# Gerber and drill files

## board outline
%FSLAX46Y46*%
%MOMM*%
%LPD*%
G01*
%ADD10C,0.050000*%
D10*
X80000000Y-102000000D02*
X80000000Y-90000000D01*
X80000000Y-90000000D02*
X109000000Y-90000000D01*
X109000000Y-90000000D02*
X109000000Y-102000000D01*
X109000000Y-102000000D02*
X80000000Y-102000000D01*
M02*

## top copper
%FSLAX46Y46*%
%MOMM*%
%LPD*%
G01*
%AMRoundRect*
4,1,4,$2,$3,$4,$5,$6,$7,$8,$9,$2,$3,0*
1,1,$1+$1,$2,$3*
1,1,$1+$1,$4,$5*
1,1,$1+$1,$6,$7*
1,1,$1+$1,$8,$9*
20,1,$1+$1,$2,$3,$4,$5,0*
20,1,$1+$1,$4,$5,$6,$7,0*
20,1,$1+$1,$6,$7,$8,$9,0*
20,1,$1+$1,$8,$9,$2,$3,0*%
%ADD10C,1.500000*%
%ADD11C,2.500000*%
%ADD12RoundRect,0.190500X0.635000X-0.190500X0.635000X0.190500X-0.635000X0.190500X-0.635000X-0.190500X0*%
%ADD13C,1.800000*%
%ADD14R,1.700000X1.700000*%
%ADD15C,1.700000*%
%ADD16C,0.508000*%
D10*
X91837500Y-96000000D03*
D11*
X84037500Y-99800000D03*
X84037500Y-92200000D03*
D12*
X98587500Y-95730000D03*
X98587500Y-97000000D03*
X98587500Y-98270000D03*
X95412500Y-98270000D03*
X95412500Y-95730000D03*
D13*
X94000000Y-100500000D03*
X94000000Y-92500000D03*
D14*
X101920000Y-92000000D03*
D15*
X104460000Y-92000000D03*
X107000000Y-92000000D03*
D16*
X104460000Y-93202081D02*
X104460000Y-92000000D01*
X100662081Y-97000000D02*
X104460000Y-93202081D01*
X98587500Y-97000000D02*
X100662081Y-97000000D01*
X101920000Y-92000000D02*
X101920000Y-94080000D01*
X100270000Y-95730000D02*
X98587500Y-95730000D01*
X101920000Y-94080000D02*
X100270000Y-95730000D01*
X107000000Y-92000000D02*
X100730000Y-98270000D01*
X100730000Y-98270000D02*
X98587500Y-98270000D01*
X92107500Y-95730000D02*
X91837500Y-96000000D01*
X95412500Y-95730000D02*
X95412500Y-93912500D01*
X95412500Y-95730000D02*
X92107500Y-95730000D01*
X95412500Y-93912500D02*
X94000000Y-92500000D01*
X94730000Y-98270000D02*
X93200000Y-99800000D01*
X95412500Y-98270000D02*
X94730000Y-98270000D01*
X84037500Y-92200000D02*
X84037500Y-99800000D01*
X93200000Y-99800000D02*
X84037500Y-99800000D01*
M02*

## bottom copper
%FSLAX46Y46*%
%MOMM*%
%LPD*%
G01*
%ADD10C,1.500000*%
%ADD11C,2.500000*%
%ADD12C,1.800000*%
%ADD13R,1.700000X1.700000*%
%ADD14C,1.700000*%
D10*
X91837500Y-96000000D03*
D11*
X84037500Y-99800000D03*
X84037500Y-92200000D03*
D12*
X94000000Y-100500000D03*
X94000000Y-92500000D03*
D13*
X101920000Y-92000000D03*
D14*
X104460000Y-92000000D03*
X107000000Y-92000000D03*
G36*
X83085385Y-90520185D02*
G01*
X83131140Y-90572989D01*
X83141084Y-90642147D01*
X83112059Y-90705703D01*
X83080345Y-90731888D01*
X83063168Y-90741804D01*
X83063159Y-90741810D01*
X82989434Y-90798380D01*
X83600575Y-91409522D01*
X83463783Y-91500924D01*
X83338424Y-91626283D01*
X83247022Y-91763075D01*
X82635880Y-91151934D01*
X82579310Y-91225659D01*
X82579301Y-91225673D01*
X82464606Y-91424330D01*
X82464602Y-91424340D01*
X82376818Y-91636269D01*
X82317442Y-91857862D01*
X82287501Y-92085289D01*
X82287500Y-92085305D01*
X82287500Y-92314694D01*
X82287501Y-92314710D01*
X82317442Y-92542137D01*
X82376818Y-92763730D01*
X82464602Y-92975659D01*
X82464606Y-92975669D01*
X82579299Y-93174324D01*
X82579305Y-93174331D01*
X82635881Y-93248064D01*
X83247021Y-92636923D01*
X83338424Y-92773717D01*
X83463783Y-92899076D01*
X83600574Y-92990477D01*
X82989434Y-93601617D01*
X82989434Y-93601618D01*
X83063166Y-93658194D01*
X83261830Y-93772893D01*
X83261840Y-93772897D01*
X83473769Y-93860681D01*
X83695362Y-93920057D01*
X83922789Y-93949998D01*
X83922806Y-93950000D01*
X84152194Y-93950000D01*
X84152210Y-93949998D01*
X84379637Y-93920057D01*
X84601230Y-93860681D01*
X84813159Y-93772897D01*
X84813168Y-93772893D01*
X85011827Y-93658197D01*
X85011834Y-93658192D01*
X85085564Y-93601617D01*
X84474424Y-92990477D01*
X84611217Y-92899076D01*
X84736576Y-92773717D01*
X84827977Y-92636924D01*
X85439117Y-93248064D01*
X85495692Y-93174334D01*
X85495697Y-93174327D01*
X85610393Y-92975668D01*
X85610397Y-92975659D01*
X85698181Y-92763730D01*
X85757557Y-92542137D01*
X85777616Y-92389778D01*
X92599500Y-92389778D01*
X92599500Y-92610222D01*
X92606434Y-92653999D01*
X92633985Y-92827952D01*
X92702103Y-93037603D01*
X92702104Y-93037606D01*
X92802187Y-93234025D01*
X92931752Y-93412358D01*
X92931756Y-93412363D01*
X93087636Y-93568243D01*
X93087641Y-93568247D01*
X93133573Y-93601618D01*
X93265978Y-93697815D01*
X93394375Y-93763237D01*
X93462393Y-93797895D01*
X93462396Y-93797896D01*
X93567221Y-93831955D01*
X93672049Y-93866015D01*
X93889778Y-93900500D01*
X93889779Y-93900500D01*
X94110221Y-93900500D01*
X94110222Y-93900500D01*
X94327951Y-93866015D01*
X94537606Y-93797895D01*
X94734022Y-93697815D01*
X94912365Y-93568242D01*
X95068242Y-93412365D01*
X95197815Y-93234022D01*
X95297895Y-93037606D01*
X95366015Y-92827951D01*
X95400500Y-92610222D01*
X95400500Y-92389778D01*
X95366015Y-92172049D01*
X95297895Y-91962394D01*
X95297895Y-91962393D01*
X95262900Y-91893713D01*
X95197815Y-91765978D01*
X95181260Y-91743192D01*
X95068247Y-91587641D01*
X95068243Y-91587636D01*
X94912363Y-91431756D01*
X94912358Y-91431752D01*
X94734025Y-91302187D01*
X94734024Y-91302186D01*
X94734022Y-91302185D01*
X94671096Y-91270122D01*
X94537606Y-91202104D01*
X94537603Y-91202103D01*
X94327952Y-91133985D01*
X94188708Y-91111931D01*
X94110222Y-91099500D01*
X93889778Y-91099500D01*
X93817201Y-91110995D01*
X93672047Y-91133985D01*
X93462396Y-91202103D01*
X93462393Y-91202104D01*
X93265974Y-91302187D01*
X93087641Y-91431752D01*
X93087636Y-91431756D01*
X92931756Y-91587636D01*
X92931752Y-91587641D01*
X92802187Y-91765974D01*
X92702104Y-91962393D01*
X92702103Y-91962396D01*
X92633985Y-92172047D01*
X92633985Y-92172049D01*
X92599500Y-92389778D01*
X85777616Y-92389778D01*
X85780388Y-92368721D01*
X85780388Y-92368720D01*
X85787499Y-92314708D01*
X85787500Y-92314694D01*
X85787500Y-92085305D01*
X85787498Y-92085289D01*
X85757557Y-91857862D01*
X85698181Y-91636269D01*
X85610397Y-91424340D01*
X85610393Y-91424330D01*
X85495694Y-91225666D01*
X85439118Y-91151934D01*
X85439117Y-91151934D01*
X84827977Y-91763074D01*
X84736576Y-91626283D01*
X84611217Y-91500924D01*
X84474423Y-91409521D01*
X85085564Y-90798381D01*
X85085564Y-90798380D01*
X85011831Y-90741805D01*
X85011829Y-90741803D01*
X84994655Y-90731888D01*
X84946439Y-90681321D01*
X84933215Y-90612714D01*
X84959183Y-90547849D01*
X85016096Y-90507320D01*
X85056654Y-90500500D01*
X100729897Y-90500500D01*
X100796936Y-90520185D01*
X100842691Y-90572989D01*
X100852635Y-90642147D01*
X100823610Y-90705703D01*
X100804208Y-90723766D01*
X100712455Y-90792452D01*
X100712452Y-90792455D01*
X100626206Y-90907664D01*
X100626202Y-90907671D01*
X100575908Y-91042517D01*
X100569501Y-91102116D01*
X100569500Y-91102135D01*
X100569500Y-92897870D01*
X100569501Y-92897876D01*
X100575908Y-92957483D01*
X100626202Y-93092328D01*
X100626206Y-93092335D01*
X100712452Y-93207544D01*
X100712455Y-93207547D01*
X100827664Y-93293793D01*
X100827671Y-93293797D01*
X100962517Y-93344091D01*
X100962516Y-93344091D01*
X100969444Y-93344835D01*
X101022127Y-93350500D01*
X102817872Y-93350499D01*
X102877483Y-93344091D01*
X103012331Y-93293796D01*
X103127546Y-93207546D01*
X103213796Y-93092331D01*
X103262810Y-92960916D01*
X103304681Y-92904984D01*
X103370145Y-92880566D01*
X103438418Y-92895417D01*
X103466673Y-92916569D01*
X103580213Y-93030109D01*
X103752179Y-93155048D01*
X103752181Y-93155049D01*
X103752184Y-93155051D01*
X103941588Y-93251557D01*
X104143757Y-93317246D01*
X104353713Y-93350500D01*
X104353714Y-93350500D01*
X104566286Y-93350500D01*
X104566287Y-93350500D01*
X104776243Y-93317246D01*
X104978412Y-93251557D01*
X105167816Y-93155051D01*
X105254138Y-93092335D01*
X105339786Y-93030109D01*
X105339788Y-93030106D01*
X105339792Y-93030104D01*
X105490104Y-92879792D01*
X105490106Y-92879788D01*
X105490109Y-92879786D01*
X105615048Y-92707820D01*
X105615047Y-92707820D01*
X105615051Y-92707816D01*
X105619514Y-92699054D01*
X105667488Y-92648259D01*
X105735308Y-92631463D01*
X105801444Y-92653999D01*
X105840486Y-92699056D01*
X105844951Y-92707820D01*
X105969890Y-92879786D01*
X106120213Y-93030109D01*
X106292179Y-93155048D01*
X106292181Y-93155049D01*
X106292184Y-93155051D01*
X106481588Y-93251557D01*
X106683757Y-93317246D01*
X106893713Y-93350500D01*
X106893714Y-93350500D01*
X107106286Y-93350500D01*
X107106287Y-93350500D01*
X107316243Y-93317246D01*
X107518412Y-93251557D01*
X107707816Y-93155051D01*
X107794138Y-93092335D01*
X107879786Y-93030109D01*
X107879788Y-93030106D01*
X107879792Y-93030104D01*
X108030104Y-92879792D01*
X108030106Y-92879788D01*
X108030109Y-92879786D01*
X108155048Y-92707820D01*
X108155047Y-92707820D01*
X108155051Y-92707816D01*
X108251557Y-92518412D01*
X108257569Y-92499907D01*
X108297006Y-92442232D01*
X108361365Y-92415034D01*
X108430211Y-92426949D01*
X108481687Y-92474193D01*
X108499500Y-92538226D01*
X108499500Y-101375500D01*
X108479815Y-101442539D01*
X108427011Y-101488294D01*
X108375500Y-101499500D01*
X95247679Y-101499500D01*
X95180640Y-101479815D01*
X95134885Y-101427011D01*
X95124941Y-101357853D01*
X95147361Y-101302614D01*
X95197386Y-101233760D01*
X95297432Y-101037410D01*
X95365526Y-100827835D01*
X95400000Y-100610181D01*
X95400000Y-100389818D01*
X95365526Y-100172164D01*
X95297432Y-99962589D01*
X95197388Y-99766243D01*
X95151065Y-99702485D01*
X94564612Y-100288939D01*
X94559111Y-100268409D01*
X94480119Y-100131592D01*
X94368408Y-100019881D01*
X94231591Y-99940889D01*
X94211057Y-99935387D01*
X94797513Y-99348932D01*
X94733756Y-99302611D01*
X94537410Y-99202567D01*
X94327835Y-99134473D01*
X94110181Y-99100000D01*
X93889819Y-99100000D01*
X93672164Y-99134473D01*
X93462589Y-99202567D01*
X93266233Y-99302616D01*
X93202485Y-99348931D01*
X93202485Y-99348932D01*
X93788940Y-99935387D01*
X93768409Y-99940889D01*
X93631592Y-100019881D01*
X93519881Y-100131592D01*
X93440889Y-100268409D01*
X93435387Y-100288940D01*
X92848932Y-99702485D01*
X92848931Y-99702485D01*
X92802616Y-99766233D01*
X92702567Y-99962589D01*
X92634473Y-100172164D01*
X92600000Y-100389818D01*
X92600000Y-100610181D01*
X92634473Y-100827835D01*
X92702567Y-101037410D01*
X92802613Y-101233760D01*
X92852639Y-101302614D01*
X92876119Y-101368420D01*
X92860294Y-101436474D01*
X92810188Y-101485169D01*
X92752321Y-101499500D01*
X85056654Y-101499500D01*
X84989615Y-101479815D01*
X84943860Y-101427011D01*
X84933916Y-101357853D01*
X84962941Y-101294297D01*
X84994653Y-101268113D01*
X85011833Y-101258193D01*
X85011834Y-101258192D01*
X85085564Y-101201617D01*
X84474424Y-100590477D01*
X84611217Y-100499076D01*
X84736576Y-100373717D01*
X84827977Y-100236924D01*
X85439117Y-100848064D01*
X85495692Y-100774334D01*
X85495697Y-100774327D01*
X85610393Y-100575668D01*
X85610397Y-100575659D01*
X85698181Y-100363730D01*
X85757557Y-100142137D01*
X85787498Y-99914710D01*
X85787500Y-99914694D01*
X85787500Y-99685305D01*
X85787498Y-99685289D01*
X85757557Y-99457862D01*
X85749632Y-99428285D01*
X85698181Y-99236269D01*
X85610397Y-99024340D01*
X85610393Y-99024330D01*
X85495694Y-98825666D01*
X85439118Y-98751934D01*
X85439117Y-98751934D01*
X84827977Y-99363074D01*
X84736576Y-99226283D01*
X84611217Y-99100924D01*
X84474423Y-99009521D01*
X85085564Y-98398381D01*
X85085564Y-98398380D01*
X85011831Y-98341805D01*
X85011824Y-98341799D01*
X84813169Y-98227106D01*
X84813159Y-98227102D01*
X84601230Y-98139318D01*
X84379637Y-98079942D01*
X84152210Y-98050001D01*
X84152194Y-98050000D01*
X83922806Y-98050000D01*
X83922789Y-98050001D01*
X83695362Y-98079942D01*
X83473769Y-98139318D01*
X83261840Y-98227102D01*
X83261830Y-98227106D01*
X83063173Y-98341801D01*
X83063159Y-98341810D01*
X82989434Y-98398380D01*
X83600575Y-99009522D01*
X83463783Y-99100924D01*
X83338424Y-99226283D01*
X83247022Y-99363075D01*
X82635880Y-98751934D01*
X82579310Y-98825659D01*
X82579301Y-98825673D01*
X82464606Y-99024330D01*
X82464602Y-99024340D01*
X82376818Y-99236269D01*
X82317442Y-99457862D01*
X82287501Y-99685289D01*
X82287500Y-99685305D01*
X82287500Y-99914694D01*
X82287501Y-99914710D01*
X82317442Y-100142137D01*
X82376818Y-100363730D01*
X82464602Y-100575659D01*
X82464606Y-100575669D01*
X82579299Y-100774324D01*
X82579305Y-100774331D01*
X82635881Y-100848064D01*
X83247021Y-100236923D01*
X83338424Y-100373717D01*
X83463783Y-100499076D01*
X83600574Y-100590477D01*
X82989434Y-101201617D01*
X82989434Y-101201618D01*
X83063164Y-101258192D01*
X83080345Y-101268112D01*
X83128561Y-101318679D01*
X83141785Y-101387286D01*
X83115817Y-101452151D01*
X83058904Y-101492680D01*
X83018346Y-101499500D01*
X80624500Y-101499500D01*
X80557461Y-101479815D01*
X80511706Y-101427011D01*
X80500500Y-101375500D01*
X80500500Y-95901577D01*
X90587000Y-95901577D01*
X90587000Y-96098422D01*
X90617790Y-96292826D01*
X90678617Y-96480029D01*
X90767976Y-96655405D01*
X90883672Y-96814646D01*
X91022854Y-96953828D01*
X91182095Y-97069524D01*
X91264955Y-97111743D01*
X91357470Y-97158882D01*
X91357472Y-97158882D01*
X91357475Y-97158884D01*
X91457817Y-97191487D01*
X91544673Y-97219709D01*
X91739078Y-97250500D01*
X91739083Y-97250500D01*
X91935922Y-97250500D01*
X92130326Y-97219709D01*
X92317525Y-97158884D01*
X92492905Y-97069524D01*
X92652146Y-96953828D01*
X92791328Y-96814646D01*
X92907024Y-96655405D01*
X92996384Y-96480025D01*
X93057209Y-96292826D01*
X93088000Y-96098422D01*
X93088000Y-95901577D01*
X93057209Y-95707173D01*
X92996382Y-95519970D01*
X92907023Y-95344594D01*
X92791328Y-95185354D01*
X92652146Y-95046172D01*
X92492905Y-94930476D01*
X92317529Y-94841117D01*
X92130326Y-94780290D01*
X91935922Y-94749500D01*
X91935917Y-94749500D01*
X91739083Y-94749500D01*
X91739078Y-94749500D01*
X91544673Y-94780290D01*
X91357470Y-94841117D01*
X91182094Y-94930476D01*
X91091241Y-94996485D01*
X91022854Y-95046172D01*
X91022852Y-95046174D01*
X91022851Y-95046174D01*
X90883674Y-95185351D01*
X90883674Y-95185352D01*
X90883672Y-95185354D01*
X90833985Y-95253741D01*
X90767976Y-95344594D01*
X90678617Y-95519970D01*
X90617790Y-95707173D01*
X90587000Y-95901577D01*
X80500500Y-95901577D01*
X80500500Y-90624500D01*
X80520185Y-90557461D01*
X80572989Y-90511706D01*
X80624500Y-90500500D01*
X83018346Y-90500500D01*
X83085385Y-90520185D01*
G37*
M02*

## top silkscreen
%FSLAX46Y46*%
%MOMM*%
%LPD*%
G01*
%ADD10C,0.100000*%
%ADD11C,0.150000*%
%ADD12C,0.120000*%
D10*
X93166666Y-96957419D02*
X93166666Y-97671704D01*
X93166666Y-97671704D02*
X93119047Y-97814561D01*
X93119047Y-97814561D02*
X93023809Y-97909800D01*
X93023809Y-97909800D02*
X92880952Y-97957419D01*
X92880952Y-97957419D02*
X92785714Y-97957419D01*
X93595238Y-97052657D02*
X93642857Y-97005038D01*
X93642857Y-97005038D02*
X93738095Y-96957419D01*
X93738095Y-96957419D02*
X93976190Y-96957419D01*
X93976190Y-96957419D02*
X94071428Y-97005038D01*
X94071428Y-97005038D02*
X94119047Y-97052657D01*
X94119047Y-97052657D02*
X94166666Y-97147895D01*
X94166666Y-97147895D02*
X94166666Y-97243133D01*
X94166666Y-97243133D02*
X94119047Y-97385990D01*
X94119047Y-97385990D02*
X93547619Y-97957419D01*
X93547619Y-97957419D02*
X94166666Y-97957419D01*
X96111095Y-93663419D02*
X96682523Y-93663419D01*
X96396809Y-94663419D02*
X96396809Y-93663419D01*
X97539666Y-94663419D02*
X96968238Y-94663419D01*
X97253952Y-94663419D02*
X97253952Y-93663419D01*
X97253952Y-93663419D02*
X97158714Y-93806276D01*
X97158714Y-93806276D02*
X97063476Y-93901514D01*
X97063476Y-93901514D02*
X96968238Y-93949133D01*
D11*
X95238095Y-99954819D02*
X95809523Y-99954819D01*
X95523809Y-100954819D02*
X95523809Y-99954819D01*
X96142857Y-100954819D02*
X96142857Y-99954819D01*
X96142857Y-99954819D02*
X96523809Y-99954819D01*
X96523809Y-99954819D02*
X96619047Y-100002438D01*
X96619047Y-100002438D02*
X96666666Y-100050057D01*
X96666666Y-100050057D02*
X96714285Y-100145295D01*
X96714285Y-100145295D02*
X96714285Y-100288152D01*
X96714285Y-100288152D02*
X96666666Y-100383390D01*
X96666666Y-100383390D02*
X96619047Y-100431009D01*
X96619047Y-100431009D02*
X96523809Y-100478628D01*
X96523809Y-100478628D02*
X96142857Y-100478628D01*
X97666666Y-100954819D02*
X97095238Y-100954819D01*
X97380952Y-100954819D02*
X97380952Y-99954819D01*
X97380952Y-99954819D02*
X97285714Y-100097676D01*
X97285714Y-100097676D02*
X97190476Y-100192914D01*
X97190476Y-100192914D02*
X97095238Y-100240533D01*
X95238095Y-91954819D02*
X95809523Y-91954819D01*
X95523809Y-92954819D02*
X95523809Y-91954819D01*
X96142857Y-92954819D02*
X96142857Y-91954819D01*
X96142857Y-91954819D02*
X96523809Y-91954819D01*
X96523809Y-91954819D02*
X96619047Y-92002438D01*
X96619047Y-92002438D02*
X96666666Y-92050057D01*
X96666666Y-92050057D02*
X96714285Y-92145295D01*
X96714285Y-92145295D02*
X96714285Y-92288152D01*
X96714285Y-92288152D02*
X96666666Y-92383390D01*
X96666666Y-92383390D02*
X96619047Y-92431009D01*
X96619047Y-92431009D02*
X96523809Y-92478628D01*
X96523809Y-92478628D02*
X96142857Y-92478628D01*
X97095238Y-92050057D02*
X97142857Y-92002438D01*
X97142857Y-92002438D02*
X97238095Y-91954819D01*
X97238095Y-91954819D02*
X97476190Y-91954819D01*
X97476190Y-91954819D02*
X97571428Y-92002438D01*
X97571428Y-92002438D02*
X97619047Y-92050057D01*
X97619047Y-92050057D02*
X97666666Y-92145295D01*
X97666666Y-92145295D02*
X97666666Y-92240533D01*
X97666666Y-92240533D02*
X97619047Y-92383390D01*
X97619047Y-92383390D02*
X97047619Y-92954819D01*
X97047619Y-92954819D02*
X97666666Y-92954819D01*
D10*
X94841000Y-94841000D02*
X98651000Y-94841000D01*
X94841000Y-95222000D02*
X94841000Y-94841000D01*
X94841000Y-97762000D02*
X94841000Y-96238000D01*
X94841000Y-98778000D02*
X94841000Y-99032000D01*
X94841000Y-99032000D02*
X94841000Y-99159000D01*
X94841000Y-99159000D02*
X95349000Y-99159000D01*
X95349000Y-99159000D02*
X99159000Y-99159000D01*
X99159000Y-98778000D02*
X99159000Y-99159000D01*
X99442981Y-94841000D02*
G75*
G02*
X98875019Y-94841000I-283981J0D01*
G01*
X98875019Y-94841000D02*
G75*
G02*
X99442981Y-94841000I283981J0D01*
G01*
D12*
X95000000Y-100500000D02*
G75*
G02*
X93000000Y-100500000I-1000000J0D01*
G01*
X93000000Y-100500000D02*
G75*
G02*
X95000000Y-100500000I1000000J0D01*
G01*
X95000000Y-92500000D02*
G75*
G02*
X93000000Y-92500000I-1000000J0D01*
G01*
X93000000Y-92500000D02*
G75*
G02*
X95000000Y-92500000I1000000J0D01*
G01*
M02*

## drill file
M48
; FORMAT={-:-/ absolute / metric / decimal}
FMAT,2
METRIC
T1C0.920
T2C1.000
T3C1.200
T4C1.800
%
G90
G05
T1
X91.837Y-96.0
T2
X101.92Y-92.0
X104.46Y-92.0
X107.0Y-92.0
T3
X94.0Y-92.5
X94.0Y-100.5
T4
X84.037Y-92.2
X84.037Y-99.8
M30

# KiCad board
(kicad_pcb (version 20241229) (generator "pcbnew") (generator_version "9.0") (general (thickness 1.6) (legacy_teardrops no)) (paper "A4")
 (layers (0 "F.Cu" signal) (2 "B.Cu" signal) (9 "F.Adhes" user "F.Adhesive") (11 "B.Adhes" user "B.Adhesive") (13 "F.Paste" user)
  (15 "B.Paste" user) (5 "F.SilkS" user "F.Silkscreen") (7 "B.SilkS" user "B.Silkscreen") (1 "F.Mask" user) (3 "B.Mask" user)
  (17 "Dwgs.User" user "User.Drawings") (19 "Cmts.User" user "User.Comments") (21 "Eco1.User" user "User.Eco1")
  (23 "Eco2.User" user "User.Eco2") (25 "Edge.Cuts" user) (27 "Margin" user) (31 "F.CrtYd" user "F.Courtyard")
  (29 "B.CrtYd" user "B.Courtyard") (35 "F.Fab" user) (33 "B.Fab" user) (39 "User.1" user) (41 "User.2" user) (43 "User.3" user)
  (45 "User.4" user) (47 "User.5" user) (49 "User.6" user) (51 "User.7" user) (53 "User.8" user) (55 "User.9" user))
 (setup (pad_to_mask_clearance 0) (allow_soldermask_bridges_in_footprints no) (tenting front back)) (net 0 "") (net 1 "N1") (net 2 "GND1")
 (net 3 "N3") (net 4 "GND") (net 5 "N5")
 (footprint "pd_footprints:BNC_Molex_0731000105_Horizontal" (layer "F.Cu") (at 84.0375 96 90)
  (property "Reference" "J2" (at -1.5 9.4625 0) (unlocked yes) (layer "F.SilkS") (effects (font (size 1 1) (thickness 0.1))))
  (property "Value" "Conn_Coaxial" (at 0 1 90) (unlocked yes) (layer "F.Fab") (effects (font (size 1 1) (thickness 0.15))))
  (pad "1" thru_hole circle (at 0 7.8 90) (size 1.5 1.5) (drill 0.92) (layers "*.Cu" "*.Mask") (remove_unused_layers no) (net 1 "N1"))
  (pad "2" thru_hole circle (at -3.8 0 90) (size 2.5 2.5) (drill 1.8) (layers "*.Cu" "*.Mask") (remove_unused_layers no) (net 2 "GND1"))
  (pad "2" thru_hole circle (at 3.8 0 90) (size 2.5 2.5) (drill 1.8) (layers "*.Cu" "*.Mask") (remove_unused_layers no) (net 2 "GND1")))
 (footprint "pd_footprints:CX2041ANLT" (layer "F.Cu") (at 97 97 90)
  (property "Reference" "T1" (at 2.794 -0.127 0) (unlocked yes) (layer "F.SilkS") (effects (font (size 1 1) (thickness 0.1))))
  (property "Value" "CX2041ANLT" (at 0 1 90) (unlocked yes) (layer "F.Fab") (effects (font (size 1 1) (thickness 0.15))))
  (fp_line (start 2.159 -2.159) (end 2.159 1.651) (stroke (width 0.1) (type default)) (layer "F.SilkS"))
  (fp_line (start 1.778 -2.159) (end 2.159 -2.159) (stroke (width 0.1) (type default)) (layer "F.SilkS"))
  (fp_line (start -0.762 -2.159) (end 0.762 -2.159) (stroke (width 0.1) (type default)) (layer "F.SilkS"))
  (fp_line (start -1.778 -2.159) (end -2.032 -2.159) (stroke (width 0.1) (type default)) (layer "F.SilkS"))
  (fp_line (start -2.032 -2.159) (end -2.159 -2.159) (stroke (width 0.1) (type default)) (layer "F.SilkS"))
  (fp_line (start -2.159 -2.159) (end -2.159 -1.651) (stroke (width 0.1) (type default)) (layer "F.SilkS"))
  (fp_line (start -2.159 -1.651) (end -2.159 2.159) (stroke (width 0.1) (type default)) (layer "F.SilkS"))
  (fp_line (start -1.778 2.159) (end -2.159 2.159) (stroke (width 0.1) (type default)) (layer "F.SilkS"))
  (fp_circle (center 2.159 2.159) (end 2.286 1.905) (stroke (width 0.1) (type default)) (fill no) (layer "F.SilkS"))
  (pad "1" smd roundrect (at 1.27 1.5875 90) (size 0.762 1.651) (layers "F.Cu" "F.Mask" "F.Paste") (roundrect_rratio 0.25) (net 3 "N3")
   (thermal_bridge_angle 45))
  (pad "2" smd roundrect (at 0 1.5875 90) (size 0.762 1.651) (layers "F.Cu" "F.Mask" "F.Paste") (roundrect_rratio 0.25) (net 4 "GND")
   (thermal_bridge_angle 45))
  (pad "3" smd roundrect (at -1.27 1.5875 90) (size 0.762 1.651) (layers "F.Cu" "F.Mask" "F.Paste") (roundrect_rratio 0.25) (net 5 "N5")
   (thermal_bridge_angle 45))
  (pad "4" smd roundrect (at -1.27 -1.5875 90) (size 0.762 1.651) (layers "F.Cu" "F.Mask" "F.Paste") (roundrect_rratio 0.25) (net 2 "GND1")
   (thermal_bridge_angle 45))
  (pad "6" smd roundrect (at 1.27 -1.5875 90) (size 0.762 1.651) (layers "F.Cu" "F.Mask" "F.Paste") (roundrect_rratio 0.25) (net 1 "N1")
   (thermal_bridge_angle 45)))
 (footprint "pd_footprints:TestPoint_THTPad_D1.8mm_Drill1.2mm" (layer "F.Cu") (at 94 100.5)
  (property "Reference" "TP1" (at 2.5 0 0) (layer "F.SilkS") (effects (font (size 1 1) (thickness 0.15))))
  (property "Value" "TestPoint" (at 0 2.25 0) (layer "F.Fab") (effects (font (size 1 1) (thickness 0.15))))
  (fp_circle (center 0 0) (end 1 0) (stroke (width 0.12) (type solid)) (fill no) (layer "F.SilkS"))
  (pad "1" thru_hole circle (at 0 0) (size 1.8 1.8) (drill 1.2) (layers "*.Cu" "*.Mask") (remove_unused_layers no) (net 2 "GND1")))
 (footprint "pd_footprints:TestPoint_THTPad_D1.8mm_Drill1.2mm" (layer "F.Cu") (at 94 92.5)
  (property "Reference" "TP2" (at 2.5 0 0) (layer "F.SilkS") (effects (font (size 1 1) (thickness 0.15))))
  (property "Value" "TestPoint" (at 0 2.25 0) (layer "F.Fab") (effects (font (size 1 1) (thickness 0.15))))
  (fp_circle (center 0 0) (end 1 0) (stroke (width 0.12) (type solid)) (fill no) (layer "F.SilkS"))
  (pad "1" thru_hole circle (at 0 0) (size 1.8 1.8) (drill 1.2) (layers "*.Cu" "*.Mask") (remove_unused_layers no) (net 1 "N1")))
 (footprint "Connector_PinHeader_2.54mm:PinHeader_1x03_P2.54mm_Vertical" (layer "B.Cu") (at 101.92 92 -90)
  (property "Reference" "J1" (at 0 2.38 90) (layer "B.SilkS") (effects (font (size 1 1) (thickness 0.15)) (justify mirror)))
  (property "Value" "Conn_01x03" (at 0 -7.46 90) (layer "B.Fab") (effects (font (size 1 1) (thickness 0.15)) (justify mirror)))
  (pad "1" thru_hole rect (at 0 0 270) (size 1.7 1.7) (drill 1) (layers "*.Cu" "*.Mask") (remove_unused_layers no) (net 3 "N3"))
  (pad "2" thru_hole circle (at 0 -2.54 270) (size 1.7 1.7) (drill 1) (layers "*.Cu" "*.Mask") (remove_unused_layers no) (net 4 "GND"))
  (pad "3" thru_hole circle (at 0 -5.08 270) (size 1.7 1.7) (drill 1) (layers "*.Cu" "*.Mask") (remove_unused_layers no) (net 5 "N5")))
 (gr_line (start 80 102) (end 80 90) (stroke (width 0.05) (type default)) (layer "Edge.Cuts"))
 (gr_line (start 80 90) (end 109 90) (stroke (width 0.05) (type default)) (layer "Edge.Cuts"))
 (gr_line (start 109 90) (end 109 102) (stroke (width 0.05) (type default)) (layer "Edge.Cuts"))
 (gr_line (start 109 102) (end 80 102) (stroke (width 0.05) (type default)) (layer "Edge.Cuts"))
 (segment (start 104.46 93.202081) (end 104.46 92) (width 0.508) (layer "F.Cu") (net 4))
 (segment (start 100.662081 97) (end 104.46 93.202081) (width 0.508) (layer "F.Cu") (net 4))
 (segment (start 98.5875 97) (end 100.662081 97) (width 0.508) (layer "F.Cu") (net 4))
 (segment (start 101.92 92) (end 101.92 94.08) (width 0.508) (layer "F.Cu") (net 3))
 (segment (start 100.27 95.73) (end 98.5875 95.73) (width 0.508) (layer "F.Cu") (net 3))
 (segment (start 101.92 94.08) (end 100.27 95.73) (width 0.508) (layer "F.Cu") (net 3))
 (segment (start 107 92) (end 100.73 98.27) (width 0.508) (layer "F.Cu") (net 5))
 (segment (start 100.73 98.27) (end 98.5875 98.27) (width 0.508) (layer "F.Cu") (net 5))
 (segment (start 92.1075 95.73) (end 91.8375 96) (width 0.508) (layer "F.Cu") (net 1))
 (segment (start 95.4125 95.73) (end 95.4125 93.9125) (width 0.508) (layer "F.Cu") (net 1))
 (segment (start 95.4125 95.73) (end 92.1075 95.73) (width 0.508) (layer "F.Cu") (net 1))
 (segment (start 95.4125 93.9125) (end 94 92.5) (width 0.508) (layer "F.Cu") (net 1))
 (segment (start 94.73 98.27) (end 93.2 99.8) (width 0.508) (layer "F.Cu") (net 2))
 (segment (start 95.4125 98.27) (end 94.73 98.27) (width 0.508) (layer "F.Cu") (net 2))
 (segment (start 84.0375 92.2) (end 84.0375 99.8) (width 0.508) (layer "F.Cu") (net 2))
 (segment (start 93.2 99.8) (end 84.0375 99.8) (width 0.508) (layer "F.Cu") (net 2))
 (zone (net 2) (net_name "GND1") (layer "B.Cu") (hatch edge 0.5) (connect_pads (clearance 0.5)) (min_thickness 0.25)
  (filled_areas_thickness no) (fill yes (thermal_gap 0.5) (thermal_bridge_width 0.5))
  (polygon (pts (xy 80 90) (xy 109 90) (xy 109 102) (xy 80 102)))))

